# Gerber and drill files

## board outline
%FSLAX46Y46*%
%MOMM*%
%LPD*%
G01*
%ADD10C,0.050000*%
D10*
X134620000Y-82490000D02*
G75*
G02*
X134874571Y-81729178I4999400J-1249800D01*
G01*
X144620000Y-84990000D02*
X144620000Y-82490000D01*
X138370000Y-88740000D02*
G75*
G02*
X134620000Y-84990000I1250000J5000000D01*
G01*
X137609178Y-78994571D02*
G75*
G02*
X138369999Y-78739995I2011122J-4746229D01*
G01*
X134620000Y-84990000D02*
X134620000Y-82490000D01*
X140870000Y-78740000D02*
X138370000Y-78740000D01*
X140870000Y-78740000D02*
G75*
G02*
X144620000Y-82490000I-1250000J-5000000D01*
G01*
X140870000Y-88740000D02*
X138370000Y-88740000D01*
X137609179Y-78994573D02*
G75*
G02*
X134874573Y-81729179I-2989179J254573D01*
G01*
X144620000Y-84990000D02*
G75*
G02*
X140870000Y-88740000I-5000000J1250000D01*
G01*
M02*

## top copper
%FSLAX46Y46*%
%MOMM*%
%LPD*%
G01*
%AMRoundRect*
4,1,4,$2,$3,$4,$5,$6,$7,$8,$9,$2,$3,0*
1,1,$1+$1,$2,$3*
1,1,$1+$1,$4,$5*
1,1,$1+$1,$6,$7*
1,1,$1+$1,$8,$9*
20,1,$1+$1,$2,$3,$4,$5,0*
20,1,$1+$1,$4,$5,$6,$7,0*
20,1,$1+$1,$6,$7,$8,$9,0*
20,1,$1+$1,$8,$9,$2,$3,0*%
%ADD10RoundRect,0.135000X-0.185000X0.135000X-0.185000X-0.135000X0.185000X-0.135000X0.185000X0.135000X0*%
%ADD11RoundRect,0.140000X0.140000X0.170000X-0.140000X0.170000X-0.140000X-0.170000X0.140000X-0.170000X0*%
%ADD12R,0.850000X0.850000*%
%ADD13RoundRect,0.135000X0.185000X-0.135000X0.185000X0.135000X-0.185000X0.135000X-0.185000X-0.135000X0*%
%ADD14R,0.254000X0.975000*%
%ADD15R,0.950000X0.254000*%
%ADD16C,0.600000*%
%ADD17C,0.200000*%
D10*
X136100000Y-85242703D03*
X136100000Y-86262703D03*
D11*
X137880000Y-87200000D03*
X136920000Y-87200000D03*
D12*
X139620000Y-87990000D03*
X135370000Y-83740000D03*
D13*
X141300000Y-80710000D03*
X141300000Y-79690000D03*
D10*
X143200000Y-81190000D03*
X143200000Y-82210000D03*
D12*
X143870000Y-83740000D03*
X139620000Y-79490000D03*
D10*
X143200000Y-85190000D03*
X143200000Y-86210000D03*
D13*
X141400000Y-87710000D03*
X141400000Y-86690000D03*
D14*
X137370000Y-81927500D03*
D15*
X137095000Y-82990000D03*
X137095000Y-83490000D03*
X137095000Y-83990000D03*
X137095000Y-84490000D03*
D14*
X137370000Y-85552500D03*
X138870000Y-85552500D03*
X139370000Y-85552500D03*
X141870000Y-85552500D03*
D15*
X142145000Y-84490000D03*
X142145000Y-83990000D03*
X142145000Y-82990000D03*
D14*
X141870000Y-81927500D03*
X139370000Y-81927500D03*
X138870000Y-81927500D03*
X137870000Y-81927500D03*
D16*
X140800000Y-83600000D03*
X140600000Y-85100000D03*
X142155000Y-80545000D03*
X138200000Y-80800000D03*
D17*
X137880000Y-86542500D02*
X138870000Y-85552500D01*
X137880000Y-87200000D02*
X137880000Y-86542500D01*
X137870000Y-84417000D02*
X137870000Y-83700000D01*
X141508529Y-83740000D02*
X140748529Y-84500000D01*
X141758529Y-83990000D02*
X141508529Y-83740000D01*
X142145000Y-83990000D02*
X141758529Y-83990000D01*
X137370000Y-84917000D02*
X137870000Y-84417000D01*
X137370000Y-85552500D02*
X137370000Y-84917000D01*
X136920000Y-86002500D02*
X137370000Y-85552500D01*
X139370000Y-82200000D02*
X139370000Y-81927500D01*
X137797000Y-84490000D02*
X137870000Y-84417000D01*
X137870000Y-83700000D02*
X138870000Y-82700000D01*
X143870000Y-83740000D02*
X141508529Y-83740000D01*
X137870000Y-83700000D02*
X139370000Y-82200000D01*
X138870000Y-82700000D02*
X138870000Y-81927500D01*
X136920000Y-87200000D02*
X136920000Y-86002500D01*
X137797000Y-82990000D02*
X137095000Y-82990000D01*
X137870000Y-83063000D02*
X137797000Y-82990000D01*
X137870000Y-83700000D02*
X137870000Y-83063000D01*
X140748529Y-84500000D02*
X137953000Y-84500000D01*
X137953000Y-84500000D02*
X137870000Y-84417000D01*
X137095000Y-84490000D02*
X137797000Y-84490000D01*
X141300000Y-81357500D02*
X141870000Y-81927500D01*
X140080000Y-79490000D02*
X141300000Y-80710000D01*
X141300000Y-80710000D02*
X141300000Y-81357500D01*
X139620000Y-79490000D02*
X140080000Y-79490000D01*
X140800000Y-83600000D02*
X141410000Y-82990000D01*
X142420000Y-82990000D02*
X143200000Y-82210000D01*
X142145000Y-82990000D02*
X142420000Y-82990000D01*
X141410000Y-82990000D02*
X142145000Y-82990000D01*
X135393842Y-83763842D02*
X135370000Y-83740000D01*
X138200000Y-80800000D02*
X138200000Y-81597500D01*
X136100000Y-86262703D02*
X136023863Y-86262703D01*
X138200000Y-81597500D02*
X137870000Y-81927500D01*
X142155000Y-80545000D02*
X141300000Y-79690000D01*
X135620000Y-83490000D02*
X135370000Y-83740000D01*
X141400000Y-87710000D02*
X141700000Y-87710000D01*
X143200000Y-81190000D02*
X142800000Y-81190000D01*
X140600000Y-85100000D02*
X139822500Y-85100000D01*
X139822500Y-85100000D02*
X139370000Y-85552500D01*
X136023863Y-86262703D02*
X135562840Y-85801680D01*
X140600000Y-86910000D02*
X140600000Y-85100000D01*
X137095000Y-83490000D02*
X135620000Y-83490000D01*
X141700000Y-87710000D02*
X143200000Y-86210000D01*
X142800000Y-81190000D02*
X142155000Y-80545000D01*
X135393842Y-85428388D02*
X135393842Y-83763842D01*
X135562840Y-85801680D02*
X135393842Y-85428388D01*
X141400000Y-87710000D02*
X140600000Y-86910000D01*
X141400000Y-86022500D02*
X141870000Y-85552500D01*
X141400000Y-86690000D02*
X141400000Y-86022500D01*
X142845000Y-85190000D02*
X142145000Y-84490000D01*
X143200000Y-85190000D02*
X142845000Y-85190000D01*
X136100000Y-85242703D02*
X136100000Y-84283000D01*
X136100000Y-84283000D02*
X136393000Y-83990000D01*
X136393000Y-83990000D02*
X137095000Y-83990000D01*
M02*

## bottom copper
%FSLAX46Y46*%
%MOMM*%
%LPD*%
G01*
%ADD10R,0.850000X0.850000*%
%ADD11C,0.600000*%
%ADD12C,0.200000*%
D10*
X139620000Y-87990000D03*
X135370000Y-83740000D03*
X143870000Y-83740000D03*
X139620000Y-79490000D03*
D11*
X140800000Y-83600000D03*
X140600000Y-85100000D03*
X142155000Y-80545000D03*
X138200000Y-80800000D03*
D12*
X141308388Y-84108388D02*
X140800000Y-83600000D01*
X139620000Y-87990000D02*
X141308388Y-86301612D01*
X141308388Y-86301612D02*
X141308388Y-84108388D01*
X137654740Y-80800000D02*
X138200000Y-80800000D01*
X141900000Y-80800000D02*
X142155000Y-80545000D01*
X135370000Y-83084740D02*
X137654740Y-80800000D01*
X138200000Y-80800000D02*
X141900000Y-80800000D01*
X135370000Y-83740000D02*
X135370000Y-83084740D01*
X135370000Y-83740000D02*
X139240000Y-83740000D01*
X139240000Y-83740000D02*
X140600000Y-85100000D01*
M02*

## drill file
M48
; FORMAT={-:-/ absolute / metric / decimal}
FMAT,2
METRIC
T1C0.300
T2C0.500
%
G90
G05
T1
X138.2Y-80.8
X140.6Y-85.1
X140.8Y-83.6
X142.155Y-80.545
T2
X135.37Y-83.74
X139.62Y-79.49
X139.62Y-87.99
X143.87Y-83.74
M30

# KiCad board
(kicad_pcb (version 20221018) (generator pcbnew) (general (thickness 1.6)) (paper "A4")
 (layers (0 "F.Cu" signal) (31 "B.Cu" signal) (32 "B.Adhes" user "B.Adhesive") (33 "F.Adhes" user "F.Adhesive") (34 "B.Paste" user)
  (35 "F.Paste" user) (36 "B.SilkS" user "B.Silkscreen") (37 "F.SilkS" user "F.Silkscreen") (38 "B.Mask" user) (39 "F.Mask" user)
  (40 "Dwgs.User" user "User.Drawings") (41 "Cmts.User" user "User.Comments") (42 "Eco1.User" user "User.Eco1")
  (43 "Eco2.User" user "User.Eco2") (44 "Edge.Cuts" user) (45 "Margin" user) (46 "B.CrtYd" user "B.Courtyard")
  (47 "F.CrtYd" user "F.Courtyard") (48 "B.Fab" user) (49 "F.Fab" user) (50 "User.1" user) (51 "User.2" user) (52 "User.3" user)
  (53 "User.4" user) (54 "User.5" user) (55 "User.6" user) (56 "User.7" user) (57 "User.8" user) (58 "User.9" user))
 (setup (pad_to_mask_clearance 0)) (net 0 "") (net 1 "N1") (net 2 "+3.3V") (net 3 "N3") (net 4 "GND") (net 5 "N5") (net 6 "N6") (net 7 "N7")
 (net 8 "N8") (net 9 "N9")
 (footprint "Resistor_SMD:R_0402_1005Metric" (layer "F.Cu") (at 136.1 85.752703 -90)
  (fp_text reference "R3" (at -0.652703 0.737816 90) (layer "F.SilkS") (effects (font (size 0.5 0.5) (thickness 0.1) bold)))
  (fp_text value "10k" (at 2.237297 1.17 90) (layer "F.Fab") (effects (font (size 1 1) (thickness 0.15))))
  (pad "1" smd roundrect (at -0.51 0 270) (size 0.54 0.64) (layers "F.Cu" "F.Paste" "F.Mask") (roundrect_rratio 0.25) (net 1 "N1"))
  (pad "2" smd roundrect (at 0.51 0 270) (size 0.54 0.64) (layers "F.Cu" "F.Paste" "F.Mask") (roundrect_rratio 0.25) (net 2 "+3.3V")))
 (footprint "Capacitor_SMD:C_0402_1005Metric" (layer "F.Cu") (at 137.4 87.2 180)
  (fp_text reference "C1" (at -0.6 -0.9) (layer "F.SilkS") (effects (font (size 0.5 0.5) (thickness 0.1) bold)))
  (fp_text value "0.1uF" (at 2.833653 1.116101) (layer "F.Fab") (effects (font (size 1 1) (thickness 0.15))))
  (pad "1" smd roundrect (at -0.48 0 180) (size 0.56 0.62) (layers "F.Cu" "F.Paste" "F.Mask") (roundrect_rratio 0.25) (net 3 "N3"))
  (pad "2" smd roundrect (at 0.48 0 180) (size 0.56 0.62) (layers "F.Cu" "F.Paste" "F.Mask") (roundrect_rratio 0.25) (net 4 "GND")))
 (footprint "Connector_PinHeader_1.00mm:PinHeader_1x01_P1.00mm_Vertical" (layer "F.Cu") (at 139.62 87.99)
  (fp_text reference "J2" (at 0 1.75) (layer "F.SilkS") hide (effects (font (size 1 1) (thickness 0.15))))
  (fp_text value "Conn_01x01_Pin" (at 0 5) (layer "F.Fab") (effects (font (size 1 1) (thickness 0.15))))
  (pad "1" thru_hole rect (at 0 0) (size 0.85 0.85) (drill 0.5) (layers "*.Cu" "*.Mask") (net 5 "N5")))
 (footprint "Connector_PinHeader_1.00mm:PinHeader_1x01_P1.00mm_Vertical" (layer "F.Cu") (at 135.37 83.74)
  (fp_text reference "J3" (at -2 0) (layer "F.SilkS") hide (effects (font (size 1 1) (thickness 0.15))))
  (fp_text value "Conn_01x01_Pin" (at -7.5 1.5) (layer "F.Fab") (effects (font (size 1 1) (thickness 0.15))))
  (pad "1" thru_hole rect (at 0 0) (size 0.85 0.85) (drill 0.5) (layers "*.Cu" "*.Mask") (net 2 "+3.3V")))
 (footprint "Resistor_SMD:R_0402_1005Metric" (layer "F.Cu") (at 141.3 80.2 90)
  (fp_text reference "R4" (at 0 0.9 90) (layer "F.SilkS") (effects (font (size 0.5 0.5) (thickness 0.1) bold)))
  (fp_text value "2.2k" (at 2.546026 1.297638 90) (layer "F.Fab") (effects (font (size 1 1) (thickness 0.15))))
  (pad "1" smd roundrect (at -0.51 0 90) (size 0.54 0.64) (layers "F.Cu" "F.Paste" "F.Mask") (roundrect_rratio 0.25) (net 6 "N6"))
  (pad "2" smd roundrect (at 0.51 0 90) (size 0.54 0.64) (layers "F.Cu" "F.Paste" "F.Mask") (roundrect_rratio 0.25) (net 2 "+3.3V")))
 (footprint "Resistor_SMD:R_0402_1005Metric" (layer "F.Cu") (at 143.2 81.7 -90)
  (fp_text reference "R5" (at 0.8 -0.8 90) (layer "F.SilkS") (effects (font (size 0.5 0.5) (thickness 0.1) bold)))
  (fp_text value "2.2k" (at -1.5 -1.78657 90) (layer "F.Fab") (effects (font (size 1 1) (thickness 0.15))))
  (pad "1" smd roundrect (at -0.51 0 270) (size 0.54 0.64) (layers "F.Cu" "F.Paste" "F.Mask") (roundrect_rratio 0.25) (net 2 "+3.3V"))
  (pad "2" smd roundrect (at 0.51 0 270) (size 0.54 0.64) (layers "F.Cu" "F.Paste" "F.Mask") (roundrect_rratio 0.25) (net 5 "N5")))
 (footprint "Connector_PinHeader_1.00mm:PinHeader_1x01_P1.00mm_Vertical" (layer "F.Cu") (at 143.87 83.74)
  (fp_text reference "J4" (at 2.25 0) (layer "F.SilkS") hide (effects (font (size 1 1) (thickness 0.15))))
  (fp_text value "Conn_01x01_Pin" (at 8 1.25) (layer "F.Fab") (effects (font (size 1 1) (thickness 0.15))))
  (pad "1" thru_hole rect (at 0 0) (size 0.85 0.85) (drill 0.5) (layers "*.Cu" "*.Mask") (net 4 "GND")))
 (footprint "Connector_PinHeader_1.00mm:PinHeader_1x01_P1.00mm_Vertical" (layer "F.Cu") (at 139.62 79.49)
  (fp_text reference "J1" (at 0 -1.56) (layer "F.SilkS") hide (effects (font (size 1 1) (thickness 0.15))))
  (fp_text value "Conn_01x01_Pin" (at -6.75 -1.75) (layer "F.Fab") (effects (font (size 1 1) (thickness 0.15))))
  (pad "1" thru_hole rect (at 0 0) (size 0.85 0.85) (drill 0.5) (layers "*.Cu" "*.Mask") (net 6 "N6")))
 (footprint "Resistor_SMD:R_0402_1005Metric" (layer "F.Cu") (at 143.2 85.7 -90)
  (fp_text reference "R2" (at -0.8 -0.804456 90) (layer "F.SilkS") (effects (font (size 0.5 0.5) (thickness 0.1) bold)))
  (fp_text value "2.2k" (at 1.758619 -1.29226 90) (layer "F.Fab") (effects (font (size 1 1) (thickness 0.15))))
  (pad "1" smd roundrect (at -0.51 0 270) (size 0.54 0.64) (layers "F.Cu" "F.Paste" "F.Mask") (roundrect_rratio 0.25) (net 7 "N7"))
  (pad "2" smd roundrect (at 0.51 0 270) (size 0.54 0.64) (layers "F.Cu" "F.Paste" "F.Mask") (roundrect_rratio 0.25) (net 2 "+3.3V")))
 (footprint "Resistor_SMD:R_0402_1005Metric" (layer "F.Cu") (at 141.4 87.2 90)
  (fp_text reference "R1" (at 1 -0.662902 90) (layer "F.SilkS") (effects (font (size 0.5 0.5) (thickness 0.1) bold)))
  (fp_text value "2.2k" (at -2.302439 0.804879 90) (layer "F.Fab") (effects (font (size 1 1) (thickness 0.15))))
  (pad "1" smd roundrect (at -0.51 0 90) (size 0.54 0.64) (layers "F.Cu" "F.Paste" "F.Mask") (roundrect_rratio 0.25) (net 2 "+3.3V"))
  (pad "2" smd roundrect (at 0.51 0 90) (size 0.54 0.64) (layers "F.Cu" "F.Paste" "F.Mask") (roundrect_rratio 0.25) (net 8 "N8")))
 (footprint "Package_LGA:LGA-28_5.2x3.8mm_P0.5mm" (layer "F.Cu") (at 139.62 83.74)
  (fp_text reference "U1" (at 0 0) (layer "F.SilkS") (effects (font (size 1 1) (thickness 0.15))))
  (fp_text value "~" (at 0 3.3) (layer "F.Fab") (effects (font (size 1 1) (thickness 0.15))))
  (pad "1" smd rect (at -2.25 -1.8125) (size 0.254 0.975) (layers "F.Cu" "F.Paste" "F.Mask") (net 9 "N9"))
  (pad "2" smd rect (at -2.525 -0.75 90) (size 0.254 0.95) (layers "F.Cu" "F.Paste" "F.Mask") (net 4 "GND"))
  (pad "3" smd rect (at -2.525 -0.25 90) (size 0.254 0.95) (layers "F.Cu" "F.Paste" "F.Mask") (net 2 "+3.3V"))
  (pad "4" smd rect (at -2.525 0.25 90) (size 0.254 0.95) (layers "F.Cu" "F.Paste" "F.Mask") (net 1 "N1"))
  (pad "5" smd rect (at -2.525 0.75 90) (size 0.254 0.95) (layers "F.Cu" "F.Paste" "F.Mask") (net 4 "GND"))
  (pad "6" smd rect (at -2.25 1.8125) (size 0.254 0.975) (layers "F.Cu" "F.Paste" "F.Mask") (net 4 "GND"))
  (pad "9" smd rect (at -0.75 1.8125) (size 0.254 0.975) (layers "F.Cu" "F.Paste" "F.Mask") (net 3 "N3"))
  (pad "10" smd rect (at -0.25 1.8125) (size 0.254 0.975) (layers "F.Cu" "F.Paste" "F.Mask") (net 2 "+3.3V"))
  (pad "15" smd rect (at 2.25 1.8125) (size 0.254 0.975) (layers "F.Cu" "F.Paste" "F.Mask") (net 8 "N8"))
  (pad "16" smd rect (at 2.525 0.75 90) (size 0.254 0.95) (layers "F.Cu" "F.Paste" "F.Mask") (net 7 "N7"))
  (pad "17" smd rect (at 2.525 0.25 90) (size 0.254 0.95) (layers "F.Cu" "F.Paste" "F.Mask") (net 4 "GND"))
  (pad "19" smd rect (at 2.525 -0.75 90) (size 0.254 0.95) (layers "F.Cu" "F.Paste" "F.Mask") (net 5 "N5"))
  (pad "20" smd rect (at 2.25 -1.8125) (size 0.254 0.975) (layers "F.Cu" "F.Paste" "F.Mask") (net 6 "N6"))
  (pad "25" smd rect (at -0.25 -1.8125) (size 0.254 0.975) (layers "F.Cu" "F.Paste" "F.Mask") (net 4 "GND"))
  (pad "26" smd rect (at -0.75 -1.8125) (size 0.254 0.975) (layers "F.Cu" "F.Paste" "F.Mask") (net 4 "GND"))
  (pad "28" smd rect (at -1.75 -1.8125) (size 0.254 0.975) (layers "F.Cu" "F.Paste" "F.Mask") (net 2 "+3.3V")))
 (gr_arc (start 134.62 82.49) (mid 134.732457 82.104627) (end 134.874571 81.729178) (stroke (width 0.05) (type default)) (layer "Edge.Cuts"))
 (gr_line (start 144.62 84.99) (end 144.62 82.49) (stroke (width 0.05) (type default)) (layer "Edge.Cuts"))
 (gr_arc (start 138.37 88.74) (mid 135.975655 87.384345) (end 134.62 84.99) (stroke (width 0.05) (type default)) (layer "Edge.Cuts"))
 (gr_arc (start 137.609178 78.994571) (mid 137.984629 78.852461) (end 138.37 78.74) (stroke (width 0.05) (type default)) (layer "Edge.Cuts"))
 (gr_line (start 134.62 84.99) (end 134.62 82.49) (stroke (width 0.05) (type default)) (layer "Edge.Cuts"))
 (gr_line (start 140.87 78.74) (end 138.37 78.74) (stroke (width 0.05) (type default)) (layer "Edge.Cuts"))
 (gr_arc (start 140.87 78.74) (mid 143.264345 80.095655) (end 144.62 82.49) (stroke (width 0.05) (type default)) (layer "Edge.Cuts"))
 (gr_line (start 140.87 88.74) (end 138.37 88.74) (stroke (width 0.05) (type default)) (layer "Edge.Cuts"))
 (gr_arc (start 137.609179 78.994573) (mid 136.74132 80.86132) (end 134.874573 81.729179) (stroke (width 0.05) (type default))
  (layer "Edge.Cuts"))
 (gr_arc (start 144.62 84.99) (mid 143.264345 87.384345) (end 140.87 88.74) (stroke (width 0.05) (type default)) (layer "Edge.Cuts"))
 (segment (start 137.88 86.5425) (end 138.87 85.5525) (width 0.2) (layer "F.Cu") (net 3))
 (segment (start 137.88 87.2) (end 137.88 86.5425) (width 0.2) (layer "F.Cu") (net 3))
 (segment (start 137.87 84.417) (end 137.87 83.7) (width 0.2) (layer "F.Cu") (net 4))
 (segment (start 141.508529 83.74) (end 140.748529 84.5) (width 0.2) (layer "F.Cu") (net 4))
 (segment (start 141.758529 83.99) (end 141.508529 83.74) (width 0.2) (layer "F.Cu") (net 4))
 (segment (start 142.145 83.99) (end 141.758529 83.99) (width 0.2) (layer "F.Cu") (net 4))
 (segment (start 137.37 84.917) (end 137.87 84.417) (width 0.2) (layer "F.Cu") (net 4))
 (segment (start 137.37 85.5525) (end 137.37 84.917) (width 0.2) (layer "F.Cu") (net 4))
 (segment (start 136.92 86.0025) (end 137.37 85.5525) (width 0.2) (layer "F.Cu") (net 4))
 (segment (start 139.37 82.2) (end 139.37 81.9275) (width 0.2) (layer "F.Cu") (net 4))
 (segment (start 137.797 84.49) (end 137.87 84.417) (width 0.2) (layer "F.Cu") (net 4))
 (segment (start 137.87 83.7) (end 138.87 82.7) (width 0.2) (layer "F.Cu") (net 4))
 (segment (start 143.87 83.74) (end 141.508529 83.74) (width 0.2) (layer "F.Cu") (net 4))
 (segment (start 137.87 83.7) (end 139.37 82.2) (width 0.2) (layer "F.Cu") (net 4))
 (segment (start 138.87 82.7) (end 138.87 81.9275) (width 0.2) (layer "F.Cu") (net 4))
 (segment (start 136.92 87.2) (end 136.92 86.0025) (width 0.2) (layer "F.Cu") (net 4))
 (segment (start 137.797 82.99) (end 137.095 82.99) (width 0.2) (layer "F.Cu") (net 4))
 (segment (start 137.87 83.063) (end 137.797 82.99) (width 0.2) (layer "F.Cu") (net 4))
 (segment (start 137.87 83.7) (end 137.87 83.063) (width 0.2) (layer "F.Cu") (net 4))
 (segment (start 140.748529 84.5) (end 137.953 84.5) (width 0.2) (layer "F.Cu") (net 4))
 (segment (start 137.953 84.5) (end 137.87 84.417) (width 0.2) (layer "F.Cu") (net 4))
 (segment (start 137.095 84.49) (end 137.797 84.49) (width 0.2) (layer "F.Cu") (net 4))
 (segment (start 141.3 81.3575) (end 141.87 81.9275) (width 0.2) (layer "F.Cu") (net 6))
 (segment (start 140.08 79.49) (end 141.3 80.71) (width 0.2) (layer "F.Cu") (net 6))
 (segment (start 141.3 80.71) (end 141.3 81.3575) (width 0.2) (layer "F.Cu") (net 6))
 (segment (start 139.62 79.49) (end 140.08 79.49) (width 0.2) (layer "F.Cu") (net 6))
 (segment (start 140.8 83.6) (end 141.41 82.99) (width 0.2) (layer "F.Cu") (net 5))
 (segment (start 142.42 82.99) (end 143.2 82.21) (width 0.2) (layer "F.Cu") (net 5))
 (segment (start 142.145 82.99) (end 142.42 82.99) (width 0.2) (layer "F.Cu") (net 5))
 (segment (start 141.41 82.99) (end 142.145 82.99) (width 0.2) (layer "F.Cu") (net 5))
 (via (at 140.8 83.6) (size 0.6) (drill 0.3) (layers "F.Cu" "B.Cu") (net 5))
 (segment (start 141.308388 84.108388) (end 140.8 83.6) (width 0.2) (layer "B.Cu") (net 5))
 (segment (start 139.62 87.99) (end 141.308388 86.301612) (width 0.2) (layer "B.Cu") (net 5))
 (segment (start 141.308388 86.301612) (end 141.308388 84.108388) (width 0.2) (layer "B.Cu") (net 5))
 (segment (start 135.393842 83.763842) (end 135.37 83.74) (width 0.2) (layer "F.Cu") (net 2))
 (segment (start 138.2 80.8) (end 138.2 81.5975) (width 0.2) (layer "F.Cu") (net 2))
 (segment (start 136.1 86.262703) (end 136.023863 86.262703) (width 0.2) (layer "F.Cu") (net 2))
 (segment (start 138.2 81.5975) (end 137.87 81.9275) (width 0.2) (layer "F.Cu") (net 2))
 (segment (start 142.155 80.545) (end 141.3 79.69) (width 0.2) (layer "F.Cu") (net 2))
 (segment (start 135.62 83.49) (end 135.37 83.74) (width 0.2) (layer "F.Cu") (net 2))
 (segment (start 141.4 87.71) (end 141.7 87.71) (width 0.2) (layer "F.Cu") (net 2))
 (segment (start 143.2 81.19) (end 142.8 81.19) (width 0.2) (layer "F.Cu") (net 2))
 (segment (start 140.6 85.1) (end 139.8225 85.1) (width 0.2) (layer "F.Cu") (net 2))
 (segment (start 139.8225 85.1) (end 139.37 85.5525) (width 0.2) (layer "F.Cu") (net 2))
 (segment (start 136.023863 86.262703) (end 135.56284 85.80168) (width 0.2) (layer "F.Cu") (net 2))
 (segment (start 140.6 86.91) (end 140.6 85.1) (width 0.2) (layer "F.Cu") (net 2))
 (segment (start 137.095 83.49) (end 135.62 83.49) (width 0.2) (layer "F.Cu") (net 2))
 (segment (start 141.7 87.71) (end 143.2 86.21) (width 0.2) (layer "F.Cu") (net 2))
 (segment (start 142.8 81.19) (end 142.155 80.545) (width 0.2) (layer "F.Cu") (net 2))
 (segment (start 135.393842 85.428388) (end 135.393842 83.763842) (width 0.2) (layer "F.Cu") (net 2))
 (segment (start 135.56284 85.80168) (end 135.393842 85.428388) (width 0.2) (layer "F.Cu") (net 2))
 (segment (start 141.4 87.71) (end 140.6 86.91) (width 0.2) (layer "F.Cu") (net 2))
 (via (at 140.6 85.1) (size 0.6) (drill 0.3) (layers "F.Cu" "B.Cu") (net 2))
 (via (at 142.155 80.545) (size 0.6) (drill 0.3) (layers "F.Cu" "B.Cu") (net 2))
 (via (at 138.2 80.8) (size 0.6) (drill 0.3) (layers "F.Cu" "B.Cu") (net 2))
 (segment (start 137.65474 80.8) (end 138.2 80.8) (width 0.2) (layer "B.Cu") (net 2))
 (segment (start 141.9 80.8) (end 142.155 80.545) (width 0.2) (layer "B.Cu") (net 2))
 (segment (start 135.37 83.08474) (end 137.65474 80.8) (width 0.2) (layer "B.Cu") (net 2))
 (segment (start 138.2 80.8) (end 141.9 80.8) (width 0.2) (layer "B.Cu") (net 2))
 (segment (start 135.37 83.74) (end 135.37 83.08474) (width 0.2) (layer "B.Cu") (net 2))
 (segment (start 135.37 83.74) (end 139.24 83.74) (width 0.2) (layer "B.Cu") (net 2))
 (segment (start 139.24 83.74) (end 140.6 85.1) (width 0.2) (layer "B.Cu") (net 2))
 (segment (start 141.4 86.0225) (end 141.87 85.5525) (width 0.2) (layer "F.Cu") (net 8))
 (segment (start 141.4 86.69) (end 141.4 86.0225) (width 0.2) (layer "F.Cu") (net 8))
 (segment (start 142.845 85.19) (end 142.145 84.49) (width 0.2) (layer "F.Cu") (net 7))
 (segment (start 143.2 85.19) (end 142.845 85.19) (width 0.2) (layer "F.Cu") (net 7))
 (segment (start 136.1 85.242703) (end 136.1 84.283) (width 0.2) (layer "F.Cu") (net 1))
 (segment (start 136.1 84.283) (end 136.393 83.99) (width 0.2) (layer "F.Cu") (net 1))
 (segment (start 136.393 83.99) (end 137.095 83.99) (width 0.2) (layer "F.Cu") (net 1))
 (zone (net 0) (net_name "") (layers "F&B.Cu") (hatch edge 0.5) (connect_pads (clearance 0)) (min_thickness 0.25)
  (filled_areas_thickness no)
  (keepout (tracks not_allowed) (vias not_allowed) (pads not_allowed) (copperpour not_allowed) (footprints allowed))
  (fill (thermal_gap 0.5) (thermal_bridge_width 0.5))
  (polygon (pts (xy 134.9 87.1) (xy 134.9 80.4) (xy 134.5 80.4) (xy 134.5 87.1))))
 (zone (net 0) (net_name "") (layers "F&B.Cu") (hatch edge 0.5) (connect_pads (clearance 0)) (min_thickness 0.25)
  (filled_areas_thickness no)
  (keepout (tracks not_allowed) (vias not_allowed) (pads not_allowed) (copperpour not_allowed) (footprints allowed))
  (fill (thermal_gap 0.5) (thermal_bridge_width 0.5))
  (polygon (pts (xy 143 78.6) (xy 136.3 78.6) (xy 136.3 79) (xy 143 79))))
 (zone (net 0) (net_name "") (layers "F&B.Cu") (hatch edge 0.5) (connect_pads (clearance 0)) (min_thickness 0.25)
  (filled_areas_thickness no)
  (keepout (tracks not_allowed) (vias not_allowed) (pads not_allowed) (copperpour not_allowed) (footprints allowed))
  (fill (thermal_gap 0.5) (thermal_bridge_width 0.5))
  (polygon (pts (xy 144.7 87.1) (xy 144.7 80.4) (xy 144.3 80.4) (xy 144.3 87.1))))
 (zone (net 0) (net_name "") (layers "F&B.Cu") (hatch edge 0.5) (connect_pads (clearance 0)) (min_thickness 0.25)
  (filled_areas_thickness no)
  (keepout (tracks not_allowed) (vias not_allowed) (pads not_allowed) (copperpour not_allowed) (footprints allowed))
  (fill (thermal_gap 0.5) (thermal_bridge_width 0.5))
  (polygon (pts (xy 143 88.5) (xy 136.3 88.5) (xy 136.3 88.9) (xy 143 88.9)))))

